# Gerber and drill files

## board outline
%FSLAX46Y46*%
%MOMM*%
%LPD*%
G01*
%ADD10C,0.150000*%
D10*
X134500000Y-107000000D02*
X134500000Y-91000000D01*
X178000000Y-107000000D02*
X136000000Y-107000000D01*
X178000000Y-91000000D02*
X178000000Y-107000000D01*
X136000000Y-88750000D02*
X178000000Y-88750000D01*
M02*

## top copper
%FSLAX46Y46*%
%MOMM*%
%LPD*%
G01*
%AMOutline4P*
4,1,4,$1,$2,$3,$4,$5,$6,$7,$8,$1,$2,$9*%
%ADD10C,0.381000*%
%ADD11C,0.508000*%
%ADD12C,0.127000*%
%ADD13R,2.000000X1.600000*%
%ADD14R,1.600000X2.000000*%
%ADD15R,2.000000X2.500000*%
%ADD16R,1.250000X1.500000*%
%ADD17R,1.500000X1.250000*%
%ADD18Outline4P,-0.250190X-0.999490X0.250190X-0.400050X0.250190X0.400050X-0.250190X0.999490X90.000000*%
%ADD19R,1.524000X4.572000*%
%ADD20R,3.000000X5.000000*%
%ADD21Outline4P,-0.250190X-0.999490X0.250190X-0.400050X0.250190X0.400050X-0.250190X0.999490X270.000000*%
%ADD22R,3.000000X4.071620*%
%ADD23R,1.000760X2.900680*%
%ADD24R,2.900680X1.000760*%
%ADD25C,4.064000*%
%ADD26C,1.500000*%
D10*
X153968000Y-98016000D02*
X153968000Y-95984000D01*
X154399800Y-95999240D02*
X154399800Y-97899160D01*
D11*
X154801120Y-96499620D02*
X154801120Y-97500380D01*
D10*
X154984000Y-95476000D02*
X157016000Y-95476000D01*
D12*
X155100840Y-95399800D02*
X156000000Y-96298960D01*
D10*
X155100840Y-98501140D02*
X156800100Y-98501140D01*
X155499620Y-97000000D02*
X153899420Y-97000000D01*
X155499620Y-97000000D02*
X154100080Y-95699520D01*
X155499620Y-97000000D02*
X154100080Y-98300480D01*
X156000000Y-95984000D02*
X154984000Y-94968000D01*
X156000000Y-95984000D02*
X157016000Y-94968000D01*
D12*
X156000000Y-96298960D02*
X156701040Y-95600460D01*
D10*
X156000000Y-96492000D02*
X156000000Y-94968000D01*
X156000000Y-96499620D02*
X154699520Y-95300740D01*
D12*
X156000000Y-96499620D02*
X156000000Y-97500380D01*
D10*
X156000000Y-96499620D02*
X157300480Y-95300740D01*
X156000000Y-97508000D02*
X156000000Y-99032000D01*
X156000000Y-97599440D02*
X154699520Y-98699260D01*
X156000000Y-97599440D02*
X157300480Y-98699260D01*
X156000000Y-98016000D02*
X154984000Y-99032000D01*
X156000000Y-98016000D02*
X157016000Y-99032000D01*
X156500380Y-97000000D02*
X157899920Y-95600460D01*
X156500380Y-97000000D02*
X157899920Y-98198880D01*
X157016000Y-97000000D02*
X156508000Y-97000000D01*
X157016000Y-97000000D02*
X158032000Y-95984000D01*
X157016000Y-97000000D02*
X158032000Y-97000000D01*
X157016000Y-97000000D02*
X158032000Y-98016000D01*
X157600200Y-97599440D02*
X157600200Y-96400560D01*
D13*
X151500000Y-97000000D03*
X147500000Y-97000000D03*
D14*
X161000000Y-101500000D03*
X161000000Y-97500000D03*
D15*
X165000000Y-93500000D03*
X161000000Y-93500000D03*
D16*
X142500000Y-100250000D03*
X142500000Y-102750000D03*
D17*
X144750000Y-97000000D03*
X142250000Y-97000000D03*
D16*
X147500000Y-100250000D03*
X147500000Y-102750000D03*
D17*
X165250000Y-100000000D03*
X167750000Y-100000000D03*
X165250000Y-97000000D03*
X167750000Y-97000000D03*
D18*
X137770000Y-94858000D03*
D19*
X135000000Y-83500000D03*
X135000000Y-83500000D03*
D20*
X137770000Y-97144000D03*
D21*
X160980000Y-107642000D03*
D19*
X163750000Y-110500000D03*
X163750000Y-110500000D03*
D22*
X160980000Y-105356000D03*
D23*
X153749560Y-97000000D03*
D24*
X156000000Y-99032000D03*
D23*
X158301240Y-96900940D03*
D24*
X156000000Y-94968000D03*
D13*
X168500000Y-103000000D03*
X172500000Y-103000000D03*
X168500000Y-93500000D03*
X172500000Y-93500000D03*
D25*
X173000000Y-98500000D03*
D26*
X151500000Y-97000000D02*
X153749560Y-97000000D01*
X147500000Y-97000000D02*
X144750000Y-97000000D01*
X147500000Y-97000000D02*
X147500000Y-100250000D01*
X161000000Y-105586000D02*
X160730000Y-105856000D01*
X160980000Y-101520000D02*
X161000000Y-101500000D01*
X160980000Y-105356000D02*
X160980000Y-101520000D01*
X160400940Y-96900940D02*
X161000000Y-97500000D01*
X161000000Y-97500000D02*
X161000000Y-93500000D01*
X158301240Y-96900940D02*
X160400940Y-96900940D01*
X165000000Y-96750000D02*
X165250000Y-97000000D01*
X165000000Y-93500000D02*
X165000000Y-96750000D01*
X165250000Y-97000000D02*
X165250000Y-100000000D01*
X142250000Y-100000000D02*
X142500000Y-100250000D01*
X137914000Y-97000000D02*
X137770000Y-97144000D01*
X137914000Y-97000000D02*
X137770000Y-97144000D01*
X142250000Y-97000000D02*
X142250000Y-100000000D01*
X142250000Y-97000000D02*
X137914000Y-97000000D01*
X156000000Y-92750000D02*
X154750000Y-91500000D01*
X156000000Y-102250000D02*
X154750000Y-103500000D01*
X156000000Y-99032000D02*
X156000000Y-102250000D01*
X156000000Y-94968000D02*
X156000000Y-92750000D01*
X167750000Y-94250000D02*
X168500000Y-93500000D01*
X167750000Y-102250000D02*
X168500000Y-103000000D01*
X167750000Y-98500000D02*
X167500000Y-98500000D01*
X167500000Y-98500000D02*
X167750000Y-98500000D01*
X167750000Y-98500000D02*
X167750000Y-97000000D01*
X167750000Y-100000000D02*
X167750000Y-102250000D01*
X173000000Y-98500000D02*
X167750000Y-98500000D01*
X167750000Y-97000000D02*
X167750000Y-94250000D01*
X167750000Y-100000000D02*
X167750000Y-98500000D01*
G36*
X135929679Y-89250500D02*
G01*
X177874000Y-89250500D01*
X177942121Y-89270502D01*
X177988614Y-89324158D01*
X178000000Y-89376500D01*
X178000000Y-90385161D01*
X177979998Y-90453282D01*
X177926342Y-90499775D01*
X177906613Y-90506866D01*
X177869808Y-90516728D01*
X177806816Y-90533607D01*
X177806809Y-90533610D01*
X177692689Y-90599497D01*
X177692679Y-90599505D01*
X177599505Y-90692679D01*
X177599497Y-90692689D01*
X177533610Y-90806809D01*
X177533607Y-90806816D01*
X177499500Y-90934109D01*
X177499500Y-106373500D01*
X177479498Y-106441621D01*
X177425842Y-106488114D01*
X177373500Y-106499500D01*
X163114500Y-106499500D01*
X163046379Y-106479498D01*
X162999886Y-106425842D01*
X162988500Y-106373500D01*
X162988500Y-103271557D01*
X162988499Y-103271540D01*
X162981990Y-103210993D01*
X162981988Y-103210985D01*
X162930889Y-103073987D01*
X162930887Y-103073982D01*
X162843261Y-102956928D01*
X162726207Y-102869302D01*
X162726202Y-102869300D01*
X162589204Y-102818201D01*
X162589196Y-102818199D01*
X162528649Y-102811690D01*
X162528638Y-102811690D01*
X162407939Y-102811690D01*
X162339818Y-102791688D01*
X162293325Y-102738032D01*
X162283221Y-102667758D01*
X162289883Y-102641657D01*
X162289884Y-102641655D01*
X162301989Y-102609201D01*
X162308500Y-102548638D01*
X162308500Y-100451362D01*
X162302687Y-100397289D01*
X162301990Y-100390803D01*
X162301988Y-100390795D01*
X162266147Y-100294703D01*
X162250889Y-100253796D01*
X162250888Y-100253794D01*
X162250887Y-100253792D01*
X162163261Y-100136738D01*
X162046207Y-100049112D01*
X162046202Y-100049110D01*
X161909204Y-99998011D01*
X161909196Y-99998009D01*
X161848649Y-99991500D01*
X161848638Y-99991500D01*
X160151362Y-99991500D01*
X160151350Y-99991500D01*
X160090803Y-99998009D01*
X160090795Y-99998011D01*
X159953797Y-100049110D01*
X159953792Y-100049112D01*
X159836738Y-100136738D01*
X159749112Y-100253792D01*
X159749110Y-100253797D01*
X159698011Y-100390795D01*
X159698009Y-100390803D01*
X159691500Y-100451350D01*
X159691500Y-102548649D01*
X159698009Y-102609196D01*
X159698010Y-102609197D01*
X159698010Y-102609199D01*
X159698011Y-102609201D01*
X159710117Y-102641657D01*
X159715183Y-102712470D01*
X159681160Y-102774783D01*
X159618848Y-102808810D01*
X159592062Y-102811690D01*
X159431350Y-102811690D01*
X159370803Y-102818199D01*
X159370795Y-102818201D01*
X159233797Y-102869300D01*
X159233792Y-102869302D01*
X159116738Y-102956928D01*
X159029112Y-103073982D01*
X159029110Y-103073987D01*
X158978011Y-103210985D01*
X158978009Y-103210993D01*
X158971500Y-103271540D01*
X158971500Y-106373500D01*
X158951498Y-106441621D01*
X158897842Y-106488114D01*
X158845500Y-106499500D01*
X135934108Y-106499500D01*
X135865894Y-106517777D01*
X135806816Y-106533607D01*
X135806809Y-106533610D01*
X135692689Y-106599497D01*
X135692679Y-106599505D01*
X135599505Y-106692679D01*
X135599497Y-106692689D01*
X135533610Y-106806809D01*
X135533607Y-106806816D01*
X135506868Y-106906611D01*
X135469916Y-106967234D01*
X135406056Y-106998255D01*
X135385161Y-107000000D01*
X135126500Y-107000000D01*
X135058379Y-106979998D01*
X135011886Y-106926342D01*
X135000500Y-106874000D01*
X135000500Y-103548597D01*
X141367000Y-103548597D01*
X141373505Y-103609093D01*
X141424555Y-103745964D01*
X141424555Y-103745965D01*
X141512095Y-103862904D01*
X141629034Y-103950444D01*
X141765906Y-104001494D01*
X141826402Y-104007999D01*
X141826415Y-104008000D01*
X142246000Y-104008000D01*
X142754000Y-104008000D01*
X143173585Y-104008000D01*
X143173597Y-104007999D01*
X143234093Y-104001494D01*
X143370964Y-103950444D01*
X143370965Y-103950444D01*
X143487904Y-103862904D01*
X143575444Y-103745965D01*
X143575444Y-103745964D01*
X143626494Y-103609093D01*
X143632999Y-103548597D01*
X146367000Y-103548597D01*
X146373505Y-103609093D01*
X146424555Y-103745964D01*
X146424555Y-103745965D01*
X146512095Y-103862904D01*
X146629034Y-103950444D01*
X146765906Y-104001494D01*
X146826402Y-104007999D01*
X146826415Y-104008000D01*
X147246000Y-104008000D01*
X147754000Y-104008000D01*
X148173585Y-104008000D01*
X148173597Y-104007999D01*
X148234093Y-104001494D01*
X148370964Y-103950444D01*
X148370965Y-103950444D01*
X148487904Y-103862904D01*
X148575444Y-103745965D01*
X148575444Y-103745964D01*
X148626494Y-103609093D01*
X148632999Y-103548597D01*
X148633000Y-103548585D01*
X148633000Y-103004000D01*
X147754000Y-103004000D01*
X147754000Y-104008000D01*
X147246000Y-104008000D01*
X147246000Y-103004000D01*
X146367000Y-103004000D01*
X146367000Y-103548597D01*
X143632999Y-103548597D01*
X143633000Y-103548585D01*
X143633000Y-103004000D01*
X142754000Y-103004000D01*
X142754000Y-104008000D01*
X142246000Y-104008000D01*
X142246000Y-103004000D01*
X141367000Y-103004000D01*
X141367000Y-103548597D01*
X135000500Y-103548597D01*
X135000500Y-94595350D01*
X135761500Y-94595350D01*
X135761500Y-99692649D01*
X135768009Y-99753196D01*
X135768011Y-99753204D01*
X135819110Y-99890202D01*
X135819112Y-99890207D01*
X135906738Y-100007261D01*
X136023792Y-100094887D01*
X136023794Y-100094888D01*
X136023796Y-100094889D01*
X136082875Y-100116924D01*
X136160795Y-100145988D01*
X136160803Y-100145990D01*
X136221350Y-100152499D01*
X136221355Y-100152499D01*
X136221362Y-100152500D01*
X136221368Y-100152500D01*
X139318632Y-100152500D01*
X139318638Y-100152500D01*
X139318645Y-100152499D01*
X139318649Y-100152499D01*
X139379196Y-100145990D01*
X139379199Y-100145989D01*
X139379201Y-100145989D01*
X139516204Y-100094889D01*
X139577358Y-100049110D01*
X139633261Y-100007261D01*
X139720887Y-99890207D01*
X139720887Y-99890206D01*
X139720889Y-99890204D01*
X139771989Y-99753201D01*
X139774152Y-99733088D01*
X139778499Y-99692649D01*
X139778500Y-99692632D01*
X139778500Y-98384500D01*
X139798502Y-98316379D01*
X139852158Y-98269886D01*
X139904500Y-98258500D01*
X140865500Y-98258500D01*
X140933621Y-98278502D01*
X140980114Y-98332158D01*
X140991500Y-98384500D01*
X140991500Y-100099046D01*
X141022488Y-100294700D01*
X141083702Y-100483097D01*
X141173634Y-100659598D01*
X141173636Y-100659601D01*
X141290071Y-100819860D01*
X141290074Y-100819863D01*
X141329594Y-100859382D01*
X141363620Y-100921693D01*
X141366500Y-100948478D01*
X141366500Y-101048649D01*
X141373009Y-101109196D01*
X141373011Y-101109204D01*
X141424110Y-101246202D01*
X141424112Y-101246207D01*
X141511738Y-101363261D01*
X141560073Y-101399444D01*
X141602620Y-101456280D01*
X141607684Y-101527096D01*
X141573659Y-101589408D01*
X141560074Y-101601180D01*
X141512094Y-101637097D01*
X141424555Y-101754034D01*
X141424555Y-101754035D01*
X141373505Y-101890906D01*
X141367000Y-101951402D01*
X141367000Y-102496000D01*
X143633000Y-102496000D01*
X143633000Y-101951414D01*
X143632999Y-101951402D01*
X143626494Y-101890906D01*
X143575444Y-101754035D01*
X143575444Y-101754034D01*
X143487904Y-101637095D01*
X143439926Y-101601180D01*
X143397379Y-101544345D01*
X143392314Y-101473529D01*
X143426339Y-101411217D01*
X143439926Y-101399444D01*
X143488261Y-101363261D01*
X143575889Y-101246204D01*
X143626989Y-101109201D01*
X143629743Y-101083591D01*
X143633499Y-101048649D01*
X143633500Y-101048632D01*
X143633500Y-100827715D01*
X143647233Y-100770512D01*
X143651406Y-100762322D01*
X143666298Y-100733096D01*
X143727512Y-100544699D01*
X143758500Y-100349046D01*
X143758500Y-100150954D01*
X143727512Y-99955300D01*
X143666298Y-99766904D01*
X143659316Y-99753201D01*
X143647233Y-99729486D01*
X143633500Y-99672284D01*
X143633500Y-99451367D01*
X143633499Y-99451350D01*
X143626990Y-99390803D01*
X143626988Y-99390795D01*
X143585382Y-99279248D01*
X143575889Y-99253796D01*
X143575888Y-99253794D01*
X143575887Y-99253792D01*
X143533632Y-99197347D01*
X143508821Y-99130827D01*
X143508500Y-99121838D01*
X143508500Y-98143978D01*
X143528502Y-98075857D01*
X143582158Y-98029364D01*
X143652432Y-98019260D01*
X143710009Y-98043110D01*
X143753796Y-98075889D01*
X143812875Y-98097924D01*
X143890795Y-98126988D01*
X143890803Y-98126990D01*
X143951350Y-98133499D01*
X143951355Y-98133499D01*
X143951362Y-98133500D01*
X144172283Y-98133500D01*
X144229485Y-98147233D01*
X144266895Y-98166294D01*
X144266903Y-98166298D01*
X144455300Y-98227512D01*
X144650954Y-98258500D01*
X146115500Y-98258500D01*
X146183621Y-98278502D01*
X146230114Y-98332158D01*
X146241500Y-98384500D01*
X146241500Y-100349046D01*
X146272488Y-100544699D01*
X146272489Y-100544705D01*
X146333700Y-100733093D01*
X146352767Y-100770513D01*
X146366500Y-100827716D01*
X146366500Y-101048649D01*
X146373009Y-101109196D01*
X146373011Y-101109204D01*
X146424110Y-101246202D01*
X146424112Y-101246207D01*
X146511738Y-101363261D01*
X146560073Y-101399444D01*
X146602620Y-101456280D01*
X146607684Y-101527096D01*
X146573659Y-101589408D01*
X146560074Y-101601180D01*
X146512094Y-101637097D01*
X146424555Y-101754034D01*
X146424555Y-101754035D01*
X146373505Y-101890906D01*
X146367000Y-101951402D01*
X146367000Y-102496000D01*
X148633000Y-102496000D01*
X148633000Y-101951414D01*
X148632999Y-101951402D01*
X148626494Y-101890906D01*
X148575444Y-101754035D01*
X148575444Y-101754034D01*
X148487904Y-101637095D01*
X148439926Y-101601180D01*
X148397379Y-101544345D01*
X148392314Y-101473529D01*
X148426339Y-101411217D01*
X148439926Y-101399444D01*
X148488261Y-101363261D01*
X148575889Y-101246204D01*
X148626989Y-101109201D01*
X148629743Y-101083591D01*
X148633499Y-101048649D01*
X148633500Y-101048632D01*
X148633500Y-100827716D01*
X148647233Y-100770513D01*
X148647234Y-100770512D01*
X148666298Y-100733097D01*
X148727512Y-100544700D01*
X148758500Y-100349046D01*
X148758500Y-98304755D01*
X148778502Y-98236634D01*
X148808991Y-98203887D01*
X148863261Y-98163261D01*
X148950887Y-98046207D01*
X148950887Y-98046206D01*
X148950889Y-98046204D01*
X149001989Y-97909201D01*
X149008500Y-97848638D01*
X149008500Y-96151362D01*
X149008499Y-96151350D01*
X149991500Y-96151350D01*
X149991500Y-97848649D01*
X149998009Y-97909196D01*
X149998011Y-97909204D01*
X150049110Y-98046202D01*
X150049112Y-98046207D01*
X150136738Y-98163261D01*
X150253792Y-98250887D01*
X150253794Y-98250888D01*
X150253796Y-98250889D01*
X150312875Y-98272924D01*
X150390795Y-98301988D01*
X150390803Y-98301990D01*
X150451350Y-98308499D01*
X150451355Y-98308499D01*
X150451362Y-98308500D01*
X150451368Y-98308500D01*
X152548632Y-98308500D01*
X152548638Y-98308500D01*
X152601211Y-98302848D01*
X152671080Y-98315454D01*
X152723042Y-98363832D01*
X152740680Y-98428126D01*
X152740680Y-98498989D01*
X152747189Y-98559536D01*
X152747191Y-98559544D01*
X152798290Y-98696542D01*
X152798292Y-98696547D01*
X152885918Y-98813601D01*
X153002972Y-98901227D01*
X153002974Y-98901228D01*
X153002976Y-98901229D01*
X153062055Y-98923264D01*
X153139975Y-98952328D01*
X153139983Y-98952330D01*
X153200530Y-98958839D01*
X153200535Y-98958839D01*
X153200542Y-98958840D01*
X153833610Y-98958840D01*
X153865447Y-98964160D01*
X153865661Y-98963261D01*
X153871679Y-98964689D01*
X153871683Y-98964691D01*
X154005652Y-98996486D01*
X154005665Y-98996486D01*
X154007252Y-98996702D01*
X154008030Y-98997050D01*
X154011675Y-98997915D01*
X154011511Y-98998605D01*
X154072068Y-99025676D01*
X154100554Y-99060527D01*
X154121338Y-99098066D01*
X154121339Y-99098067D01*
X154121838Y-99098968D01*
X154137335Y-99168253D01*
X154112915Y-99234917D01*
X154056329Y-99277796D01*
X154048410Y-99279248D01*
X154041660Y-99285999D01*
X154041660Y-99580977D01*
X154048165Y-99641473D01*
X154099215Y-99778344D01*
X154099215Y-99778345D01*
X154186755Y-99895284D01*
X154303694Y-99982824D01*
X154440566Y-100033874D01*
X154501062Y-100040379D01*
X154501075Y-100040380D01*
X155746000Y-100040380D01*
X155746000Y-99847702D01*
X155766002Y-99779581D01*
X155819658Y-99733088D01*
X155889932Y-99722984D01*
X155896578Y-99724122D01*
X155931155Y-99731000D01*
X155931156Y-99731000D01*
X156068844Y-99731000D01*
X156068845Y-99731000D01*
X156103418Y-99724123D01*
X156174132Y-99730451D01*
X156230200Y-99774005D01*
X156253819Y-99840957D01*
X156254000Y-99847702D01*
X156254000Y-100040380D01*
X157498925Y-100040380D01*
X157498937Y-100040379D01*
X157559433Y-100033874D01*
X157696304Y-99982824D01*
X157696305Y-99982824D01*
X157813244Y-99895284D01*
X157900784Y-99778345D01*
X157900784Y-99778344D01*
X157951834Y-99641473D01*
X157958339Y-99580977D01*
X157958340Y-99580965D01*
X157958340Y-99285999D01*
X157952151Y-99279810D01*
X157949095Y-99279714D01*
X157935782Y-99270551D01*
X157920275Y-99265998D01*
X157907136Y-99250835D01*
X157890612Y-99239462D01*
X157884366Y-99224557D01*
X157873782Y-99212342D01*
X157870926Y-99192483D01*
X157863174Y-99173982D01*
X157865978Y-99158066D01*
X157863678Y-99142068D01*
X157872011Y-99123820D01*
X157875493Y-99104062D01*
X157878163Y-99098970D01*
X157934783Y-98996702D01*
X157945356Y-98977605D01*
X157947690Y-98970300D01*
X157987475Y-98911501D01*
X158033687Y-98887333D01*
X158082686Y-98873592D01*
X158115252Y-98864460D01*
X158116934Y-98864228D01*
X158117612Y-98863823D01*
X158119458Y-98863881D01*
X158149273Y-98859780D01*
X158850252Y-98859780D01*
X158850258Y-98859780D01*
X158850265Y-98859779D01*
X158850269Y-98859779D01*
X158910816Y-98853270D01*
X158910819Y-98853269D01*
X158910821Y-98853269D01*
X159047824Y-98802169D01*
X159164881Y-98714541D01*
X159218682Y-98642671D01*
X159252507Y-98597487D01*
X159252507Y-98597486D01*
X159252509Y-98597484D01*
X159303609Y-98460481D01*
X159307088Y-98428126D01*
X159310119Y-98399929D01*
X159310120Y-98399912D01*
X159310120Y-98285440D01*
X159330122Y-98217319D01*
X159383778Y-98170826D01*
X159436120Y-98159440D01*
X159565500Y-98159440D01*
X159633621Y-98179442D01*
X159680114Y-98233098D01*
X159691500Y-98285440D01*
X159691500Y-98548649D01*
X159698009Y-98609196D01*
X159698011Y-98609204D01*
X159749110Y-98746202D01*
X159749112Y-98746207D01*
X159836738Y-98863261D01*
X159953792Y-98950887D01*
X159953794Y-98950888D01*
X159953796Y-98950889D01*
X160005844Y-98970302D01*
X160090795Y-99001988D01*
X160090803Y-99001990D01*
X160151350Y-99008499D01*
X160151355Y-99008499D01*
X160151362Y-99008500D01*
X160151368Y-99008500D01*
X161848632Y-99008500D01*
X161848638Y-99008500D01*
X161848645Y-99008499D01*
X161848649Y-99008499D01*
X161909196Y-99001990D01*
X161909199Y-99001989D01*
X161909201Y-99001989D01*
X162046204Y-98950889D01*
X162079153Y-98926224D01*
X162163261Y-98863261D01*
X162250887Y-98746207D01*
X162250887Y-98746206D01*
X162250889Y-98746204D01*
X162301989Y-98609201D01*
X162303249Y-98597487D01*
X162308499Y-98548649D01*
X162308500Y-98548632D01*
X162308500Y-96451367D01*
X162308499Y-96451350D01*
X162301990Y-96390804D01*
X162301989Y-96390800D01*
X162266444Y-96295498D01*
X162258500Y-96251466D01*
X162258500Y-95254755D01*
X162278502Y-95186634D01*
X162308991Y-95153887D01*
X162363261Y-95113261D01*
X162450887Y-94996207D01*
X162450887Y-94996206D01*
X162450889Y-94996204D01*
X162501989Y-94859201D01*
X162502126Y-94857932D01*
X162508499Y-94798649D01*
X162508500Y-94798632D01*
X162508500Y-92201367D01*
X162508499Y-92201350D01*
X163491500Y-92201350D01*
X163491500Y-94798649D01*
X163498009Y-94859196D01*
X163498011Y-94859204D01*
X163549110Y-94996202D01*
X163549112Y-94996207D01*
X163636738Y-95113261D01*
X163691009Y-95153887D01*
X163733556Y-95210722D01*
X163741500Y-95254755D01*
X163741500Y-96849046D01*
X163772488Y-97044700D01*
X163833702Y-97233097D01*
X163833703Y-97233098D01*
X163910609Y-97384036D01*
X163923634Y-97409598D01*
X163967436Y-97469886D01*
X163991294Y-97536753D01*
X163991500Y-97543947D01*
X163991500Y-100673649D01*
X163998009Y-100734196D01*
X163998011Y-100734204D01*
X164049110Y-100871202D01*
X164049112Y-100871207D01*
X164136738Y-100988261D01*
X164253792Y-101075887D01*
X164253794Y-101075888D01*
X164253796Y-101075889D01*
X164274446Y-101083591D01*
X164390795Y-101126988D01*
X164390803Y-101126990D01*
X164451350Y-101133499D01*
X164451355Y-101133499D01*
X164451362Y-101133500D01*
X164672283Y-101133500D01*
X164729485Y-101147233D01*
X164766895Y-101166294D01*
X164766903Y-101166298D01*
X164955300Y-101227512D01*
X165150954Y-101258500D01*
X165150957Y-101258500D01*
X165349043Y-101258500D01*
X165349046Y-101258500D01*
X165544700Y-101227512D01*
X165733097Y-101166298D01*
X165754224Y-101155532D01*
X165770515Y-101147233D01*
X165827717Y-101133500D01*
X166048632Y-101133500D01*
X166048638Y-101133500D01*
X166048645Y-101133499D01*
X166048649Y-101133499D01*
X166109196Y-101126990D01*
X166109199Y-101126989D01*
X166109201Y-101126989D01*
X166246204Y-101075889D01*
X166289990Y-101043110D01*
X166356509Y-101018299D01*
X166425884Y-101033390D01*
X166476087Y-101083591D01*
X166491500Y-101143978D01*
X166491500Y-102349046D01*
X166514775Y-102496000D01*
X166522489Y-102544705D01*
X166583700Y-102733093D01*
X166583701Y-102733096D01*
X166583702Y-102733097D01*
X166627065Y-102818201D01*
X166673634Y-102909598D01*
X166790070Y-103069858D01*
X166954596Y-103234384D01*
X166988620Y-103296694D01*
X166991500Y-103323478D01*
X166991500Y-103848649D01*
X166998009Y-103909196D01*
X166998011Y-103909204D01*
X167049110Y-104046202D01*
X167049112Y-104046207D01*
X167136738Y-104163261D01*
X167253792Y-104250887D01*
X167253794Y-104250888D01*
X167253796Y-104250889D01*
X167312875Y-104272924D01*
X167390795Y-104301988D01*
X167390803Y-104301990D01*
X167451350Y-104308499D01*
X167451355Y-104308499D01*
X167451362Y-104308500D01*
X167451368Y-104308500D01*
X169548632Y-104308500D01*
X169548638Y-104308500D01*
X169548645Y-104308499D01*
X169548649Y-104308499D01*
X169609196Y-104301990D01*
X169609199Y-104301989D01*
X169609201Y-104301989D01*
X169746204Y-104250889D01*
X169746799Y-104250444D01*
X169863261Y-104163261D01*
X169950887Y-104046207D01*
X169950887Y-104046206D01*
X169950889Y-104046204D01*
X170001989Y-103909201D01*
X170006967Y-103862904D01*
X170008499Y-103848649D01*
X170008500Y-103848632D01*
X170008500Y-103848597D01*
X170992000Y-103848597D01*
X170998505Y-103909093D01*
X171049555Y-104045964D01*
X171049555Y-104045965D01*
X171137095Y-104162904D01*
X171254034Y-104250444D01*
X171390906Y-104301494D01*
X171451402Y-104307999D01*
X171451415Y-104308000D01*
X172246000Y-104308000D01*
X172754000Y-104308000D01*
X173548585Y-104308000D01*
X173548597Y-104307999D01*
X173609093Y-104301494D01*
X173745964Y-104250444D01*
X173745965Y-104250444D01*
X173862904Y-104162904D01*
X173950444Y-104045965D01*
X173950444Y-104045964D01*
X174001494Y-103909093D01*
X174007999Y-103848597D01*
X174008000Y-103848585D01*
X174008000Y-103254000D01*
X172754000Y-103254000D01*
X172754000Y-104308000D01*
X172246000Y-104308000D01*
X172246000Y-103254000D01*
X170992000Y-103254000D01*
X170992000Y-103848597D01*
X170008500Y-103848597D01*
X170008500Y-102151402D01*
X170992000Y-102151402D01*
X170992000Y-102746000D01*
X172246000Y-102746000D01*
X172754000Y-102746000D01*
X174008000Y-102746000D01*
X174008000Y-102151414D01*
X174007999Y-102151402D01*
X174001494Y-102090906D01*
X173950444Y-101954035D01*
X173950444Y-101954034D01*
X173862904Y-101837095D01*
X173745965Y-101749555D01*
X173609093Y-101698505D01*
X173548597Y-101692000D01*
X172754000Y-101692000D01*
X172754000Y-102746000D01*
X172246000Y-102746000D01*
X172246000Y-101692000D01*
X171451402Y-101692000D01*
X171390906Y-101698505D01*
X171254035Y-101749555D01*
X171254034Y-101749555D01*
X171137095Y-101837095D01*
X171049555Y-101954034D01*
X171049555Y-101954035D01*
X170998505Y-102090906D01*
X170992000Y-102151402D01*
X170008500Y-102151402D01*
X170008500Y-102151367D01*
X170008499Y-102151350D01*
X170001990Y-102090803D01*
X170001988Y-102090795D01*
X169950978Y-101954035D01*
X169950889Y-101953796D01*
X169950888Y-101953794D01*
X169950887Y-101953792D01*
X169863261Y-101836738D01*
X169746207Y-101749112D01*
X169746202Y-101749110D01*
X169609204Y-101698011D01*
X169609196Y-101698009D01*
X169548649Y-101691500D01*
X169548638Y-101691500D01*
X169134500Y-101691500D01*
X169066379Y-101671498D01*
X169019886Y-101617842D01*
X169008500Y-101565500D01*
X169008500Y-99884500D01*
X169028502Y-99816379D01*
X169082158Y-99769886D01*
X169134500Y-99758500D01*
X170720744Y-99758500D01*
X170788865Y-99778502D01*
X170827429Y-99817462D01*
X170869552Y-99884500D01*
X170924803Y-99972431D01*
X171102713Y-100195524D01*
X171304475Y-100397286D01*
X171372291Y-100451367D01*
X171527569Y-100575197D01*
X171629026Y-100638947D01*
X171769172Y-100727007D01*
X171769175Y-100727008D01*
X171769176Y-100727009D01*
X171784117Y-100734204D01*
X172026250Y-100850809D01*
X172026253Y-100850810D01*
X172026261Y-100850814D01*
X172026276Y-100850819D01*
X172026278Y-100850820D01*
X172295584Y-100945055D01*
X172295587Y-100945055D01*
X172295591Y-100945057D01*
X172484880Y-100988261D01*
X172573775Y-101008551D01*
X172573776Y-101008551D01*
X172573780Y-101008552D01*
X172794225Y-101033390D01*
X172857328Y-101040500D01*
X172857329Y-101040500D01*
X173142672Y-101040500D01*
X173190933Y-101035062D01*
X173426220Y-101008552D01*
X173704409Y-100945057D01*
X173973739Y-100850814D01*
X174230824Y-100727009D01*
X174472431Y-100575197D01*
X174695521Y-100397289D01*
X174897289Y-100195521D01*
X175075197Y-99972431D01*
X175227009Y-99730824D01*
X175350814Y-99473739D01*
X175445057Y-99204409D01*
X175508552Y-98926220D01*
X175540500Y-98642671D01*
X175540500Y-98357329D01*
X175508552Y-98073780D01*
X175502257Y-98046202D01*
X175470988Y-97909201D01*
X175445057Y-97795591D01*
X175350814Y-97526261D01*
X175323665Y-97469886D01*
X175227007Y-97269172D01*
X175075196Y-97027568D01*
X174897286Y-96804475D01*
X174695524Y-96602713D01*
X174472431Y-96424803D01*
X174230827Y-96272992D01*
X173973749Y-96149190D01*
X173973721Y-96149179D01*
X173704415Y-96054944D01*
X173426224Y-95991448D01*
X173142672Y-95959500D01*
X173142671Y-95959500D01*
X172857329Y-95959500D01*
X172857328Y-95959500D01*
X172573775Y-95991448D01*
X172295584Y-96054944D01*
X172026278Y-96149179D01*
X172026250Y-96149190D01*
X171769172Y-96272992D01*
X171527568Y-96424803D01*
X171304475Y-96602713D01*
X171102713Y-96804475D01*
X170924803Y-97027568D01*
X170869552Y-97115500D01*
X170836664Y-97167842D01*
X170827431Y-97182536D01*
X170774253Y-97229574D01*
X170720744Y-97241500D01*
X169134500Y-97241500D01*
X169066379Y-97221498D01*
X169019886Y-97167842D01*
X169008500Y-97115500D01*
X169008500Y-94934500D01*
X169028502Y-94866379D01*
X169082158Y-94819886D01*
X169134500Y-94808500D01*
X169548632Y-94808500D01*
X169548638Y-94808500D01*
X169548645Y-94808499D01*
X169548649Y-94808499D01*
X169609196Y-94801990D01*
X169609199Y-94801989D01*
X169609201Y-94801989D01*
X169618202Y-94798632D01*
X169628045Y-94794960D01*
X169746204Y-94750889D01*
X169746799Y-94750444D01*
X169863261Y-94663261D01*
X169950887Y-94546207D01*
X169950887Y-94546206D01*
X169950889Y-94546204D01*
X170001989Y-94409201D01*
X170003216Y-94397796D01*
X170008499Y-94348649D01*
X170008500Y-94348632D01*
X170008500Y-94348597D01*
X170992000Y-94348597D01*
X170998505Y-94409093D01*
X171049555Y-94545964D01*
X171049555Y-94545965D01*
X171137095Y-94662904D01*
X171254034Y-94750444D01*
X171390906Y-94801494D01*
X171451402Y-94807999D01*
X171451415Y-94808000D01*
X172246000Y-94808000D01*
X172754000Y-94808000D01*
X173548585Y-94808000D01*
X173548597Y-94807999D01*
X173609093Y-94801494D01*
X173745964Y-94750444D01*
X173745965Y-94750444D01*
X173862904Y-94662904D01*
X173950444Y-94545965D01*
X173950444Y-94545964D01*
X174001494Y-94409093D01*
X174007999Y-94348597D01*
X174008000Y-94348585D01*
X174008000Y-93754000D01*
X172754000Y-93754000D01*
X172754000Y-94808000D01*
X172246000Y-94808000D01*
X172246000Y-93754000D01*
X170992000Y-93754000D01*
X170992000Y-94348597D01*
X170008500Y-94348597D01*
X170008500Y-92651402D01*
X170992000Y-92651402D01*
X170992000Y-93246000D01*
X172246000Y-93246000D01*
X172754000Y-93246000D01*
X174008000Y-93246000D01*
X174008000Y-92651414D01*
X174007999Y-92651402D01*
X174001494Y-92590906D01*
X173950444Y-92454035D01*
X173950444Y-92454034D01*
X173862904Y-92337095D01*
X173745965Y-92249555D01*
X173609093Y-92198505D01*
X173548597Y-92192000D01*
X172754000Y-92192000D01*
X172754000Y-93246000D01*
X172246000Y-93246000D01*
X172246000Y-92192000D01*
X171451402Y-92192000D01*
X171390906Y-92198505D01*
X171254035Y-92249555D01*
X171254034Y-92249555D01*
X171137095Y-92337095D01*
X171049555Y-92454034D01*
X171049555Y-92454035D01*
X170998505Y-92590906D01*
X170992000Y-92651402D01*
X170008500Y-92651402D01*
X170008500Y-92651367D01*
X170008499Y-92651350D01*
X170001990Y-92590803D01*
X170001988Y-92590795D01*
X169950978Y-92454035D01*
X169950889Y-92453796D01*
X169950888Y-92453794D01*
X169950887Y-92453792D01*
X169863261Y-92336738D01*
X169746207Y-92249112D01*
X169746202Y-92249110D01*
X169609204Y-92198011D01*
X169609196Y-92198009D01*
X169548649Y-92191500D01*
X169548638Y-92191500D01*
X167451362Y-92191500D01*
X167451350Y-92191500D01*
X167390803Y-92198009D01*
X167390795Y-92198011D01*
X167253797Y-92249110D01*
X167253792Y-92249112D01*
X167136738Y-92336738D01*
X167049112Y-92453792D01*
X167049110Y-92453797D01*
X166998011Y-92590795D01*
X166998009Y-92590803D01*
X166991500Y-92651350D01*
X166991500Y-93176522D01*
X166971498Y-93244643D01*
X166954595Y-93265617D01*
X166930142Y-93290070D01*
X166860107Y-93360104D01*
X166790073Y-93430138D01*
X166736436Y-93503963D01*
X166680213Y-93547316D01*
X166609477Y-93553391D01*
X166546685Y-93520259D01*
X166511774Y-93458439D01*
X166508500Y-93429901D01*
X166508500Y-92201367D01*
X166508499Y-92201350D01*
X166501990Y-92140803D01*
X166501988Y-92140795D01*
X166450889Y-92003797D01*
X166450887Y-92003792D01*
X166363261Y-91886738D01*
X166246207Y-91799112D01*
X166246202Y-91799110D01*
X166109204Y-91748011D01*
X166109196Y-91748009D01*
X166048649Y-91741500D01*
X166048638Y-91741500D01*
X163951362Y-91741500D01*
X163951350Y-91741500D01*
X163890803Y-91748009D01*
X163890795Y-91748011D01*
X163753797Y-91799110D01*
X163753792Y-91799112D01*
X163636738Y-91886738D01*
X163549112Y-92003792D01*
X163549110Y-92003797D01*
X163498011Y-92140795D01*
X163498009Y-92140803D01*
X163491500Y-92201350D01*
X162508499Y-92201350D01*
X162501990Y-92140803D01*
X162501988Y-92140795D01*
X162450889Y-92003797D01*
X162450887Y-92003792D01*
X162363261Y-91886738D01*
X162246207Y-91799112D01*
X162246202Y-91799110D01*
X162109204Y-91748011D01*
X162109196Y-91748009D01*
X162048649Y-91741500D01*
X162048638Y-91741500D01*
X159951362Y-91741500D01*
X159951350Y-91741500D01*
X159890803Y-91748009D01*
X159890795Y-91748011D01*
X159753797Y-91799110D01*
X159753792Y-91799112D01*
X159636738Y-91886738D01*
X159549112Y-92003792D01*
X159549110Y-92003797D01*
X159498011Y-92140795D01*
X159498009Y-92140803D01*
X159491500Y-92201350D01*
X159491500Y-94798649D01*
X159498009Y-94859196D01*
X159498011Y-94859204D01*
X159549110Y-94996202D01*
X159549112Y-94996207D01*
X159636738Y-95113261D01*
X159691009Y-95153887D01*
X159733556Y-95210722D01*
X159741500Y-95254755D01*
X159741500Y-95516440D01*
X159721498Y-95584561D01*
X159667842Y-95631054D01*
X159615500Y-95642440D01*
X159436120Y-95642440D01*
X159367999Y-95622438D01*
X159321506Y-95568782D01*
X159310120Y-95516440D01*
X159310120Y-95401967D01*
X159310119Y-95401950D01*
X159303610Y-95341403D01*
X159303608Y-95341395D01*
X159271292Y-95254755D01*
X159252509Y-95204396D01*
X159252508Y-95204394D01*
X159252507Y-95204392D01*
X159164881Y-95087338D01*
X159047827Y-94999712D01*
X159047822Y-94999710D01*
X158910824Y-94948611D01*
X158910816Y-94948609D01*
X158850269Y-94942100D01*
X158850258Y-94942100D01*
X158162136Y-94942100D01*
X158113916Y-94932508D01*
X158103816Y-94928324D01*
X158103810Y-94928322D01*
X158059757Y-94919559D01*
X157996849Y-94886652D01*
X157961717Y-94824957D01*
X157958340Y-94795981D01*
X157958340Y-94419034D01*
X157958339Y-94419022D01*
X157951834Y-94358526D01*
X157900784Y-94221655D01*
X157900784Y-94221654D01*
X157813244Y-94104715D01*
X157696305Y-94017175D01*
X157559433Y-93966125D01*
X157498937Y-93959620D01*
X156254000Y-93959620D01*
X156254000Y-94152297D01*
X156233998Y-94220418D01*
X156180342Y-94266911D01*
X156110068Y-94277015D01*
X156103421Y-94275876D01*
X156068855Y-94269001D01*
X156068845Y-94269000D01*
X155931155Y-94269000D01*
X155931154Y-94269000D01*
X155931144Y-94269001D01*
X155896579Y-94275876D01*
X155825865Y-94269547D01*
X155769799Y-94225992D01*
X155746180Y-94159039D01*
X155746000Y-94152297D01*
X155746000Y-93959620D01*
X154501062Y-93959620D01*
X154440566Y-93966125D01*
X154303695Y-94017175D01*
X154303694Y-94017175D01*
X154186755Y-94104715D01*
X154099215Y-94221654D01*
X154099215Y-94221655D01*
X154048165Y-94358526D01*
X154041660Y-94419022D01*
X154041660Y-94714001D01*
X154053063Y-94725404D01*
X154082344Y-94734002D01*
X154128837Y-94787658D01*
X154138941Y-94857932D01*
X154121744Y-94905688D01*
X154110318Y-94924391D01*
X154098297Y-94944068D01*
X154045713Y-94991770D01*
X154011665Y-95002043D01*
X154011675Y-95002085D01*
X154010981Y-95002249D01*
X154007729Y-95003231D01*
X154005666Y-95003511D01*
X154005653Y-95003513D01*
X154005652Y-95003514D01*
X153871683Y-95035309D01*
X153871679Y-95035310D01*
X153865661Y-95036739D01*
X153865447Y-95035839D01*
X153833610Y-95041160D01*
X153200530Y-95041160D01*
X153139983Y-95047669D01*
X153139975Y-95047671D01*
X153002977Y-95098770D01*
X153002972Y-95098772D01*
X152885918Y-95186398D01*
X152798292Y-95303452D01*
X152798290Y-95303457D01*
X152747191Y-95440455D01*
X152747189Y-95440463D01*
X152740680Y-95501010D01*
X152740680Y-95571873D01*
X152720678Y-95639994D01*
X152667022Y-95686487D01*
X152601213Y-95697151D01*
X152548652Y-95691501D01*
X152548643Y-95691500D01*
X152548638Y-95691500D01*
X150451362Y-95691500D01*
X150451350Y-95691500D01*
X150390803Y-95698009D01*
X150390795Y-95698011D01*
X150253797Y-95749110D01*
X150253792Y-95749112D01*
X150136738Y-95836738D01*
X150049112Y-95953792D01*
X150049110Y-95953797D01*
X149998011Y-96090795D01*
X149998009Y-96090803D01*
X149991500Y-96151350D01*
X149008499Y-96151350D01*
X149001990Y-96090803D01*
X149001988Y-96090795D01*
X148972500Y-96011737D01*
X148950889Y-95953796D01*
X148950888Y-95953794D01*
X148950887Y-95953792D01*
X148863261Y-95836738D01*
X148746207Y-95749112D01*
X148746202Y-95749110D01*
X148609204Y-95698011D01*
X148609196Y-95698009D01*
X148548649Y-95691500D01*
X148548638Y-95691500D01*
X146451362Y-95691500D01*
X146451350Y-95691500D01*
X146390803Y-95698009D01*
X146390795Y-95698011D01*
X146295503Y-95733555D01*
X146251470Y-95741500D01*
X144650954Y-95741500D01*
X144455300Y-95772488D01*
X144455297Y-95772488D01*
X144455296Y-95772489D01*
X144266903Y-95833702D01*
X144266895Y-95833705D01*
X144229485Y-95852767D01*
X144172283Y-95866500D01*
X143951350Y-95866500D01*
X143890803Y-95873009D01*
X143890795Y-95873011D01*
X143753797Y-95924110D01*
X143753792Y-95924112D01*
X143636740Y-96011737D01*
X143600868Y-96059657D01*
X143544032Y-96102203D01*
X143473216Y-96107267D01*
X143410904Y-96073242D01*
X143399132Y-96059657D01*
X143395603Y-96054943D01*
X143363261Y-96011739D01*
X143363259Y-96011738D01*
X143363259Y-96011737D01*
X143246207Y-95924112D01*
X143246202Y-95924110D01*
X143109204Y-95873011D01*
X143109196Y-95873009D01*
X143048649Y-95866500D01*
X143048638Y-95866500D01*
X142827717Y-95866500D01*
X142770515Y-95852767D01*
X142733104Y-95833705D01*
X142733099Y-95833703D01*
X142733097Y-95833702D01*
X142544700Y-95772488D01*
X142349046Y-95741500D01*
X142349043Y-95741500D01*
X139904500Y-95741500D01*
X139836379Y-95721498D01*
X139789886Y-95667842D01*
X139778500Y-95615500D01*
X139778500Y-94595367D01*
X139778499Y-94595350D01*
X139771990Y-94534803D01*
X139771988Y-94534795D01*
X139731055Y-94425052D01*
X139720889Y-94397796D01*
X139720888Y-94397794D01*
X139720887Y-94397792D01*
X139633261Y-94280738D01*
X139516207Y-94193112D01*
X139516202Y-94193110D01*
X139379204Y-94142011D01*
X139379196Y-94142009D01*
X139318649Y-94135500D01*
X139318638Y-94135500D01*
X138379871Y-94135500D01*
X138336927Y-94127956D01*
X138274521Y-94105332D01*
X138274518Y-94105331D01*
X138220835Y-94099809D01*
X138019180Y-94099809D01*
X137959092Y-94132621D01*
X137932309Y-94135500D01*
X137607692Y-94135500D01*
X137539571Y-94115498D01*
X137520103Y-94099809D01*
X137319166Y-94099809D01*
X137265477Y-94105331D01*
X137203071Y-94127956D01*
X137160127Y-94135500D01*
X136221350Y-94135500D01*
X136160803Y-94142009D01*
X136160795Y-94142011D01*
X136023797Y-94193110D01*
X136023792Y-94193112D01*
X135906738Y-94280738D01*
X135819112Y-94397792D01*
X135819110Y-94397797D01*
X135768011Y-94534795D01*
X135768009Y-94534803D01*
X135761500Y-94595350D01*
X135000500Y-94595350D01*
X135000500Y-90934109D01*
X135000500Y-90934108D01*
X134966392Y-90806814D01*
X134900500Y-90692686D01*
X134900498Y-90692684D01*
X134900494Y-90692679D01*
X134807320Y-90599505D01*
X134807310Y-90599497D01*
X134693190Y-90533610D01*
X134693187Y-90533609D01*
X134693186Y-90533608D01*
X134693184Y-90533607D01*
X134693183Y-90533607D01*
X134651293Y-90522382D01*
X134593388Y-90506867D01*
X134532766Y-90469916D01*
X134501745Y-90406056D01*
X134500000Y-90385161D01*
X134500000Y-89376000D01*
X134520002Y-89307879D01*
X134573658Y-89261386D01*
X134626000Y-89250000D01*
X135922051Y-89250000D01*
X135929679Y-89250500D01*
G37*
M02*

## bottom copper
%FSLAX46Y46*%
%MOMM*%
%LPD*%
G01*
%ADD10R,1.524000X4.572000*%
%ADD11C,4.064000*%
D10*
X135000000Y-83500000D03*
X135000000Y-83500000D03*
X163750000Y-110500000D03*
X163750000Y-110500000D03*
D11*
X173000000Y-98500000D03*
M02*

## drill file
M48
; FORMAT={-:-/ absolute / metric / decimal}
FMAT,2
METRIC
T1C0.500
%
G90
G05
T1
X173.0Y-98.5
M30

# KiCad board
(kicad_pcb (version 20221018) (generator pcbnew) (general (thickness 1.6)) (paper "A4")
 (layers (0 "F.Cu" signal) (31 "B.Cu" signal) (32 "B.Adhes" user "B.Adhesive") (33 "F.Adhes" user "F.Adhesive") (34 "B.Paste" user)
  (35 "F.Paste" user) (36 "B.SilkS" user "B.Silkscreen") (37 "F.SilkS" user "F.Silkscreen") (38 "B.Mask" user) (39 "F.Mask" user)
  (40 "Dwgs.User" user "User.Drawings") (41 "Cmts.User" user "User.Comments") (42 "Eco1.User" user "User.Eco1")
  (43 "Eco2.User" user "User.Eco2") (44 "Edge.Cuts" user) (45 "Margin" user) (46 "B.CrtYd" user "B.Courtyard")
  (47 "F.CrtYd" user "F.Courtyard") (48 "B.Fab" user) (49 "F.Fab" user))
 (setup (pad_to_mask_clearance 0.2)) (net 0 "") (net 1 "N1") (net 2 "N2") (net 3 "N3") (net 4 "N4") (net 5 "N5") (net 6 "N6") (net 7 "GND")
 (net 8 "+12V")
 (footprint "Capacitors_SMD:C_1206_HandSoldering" (layer "F.Cu") (at 149.5 97 180)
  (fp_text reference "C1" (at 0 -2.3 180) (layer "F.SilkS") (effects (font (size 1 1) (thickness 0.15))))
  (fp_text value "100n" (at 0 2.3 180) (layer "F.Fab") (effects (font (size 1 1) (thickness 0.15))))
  (pad "1" smd rect (at -2 0 180) (size 2 1.6) (layers "F.Cu" "F.Paste" "F.Mask") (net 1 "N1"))
  (pad "2" smd rect (at 2 0 180) (size 2 1.6) (layers "F.Cu" "F.Paste" "F.Mask") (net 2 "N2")))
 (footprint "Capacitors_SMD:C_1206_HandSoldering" (layer "F.Cu") (at 161 99.5 90)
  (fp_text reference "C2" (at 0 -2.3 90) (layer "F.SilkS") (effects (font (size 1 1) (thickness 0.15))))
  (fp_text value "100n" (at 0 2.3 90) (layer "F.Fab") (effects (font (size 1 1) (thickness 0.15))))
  (pad "1" smd rect (at -2 0 90) (size 2 1.6) (layers "F.Cu" "F.Paste" "F.Mask") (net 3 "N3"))
  (pad "2" smd rect (at 2 0 90) (size 2 1.6) (layers "F.Cu" "F.Paste" "F.Mask") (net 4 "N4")))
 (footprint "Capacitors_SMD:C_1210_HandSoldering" (layer "F.Cu") (at 163 93.5 180)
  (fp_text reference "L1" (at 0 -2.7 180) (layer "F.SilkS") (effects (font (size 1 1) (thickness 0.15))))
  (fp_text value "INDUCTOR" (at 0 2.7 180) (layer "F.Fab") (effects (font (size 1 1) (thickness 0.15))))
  (pad "1" smd rect (at -2 0 180) (size 2 2.5) (layers "F.Cu" "F.Paste" "F.Mask") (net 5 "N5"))
  (pad "2" smd rect (at 2 0 180) (size 2 2.5) (layers "F.Cu" "F.Paste" "F.Mask") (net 4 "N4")))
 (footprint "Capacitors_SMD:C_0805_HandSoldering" (layer "F.Cu") (at 142.5 101.5 -90)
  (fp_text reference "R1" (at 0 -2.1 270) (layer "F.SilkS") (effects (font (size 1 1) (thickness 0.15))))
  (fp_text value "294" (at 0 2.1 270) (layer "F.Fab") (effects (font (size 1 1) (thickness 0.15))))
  (pad "1" smd rect (at -1.25 0 270) (size 1.5 1.25) (layers "F.Cu" "F.Paste" "F.Mask") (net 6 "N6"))
  (pad "2" smd rect (at 1.25 0 270) (size 1.5 1.25) (layers "F.Cu" "F.Paste" "F.Mask") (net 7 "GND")))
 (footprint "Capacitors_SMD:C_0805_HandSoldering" (layer "F.Cu") (at 143.5 97 180)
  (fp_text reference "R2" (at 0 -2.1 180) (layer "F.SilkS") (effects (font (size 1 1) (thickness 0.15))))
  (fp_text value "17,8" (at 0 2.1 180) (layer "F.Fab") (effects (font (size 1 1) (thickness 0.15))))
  (pad "1" smd rect (at -1.25 0 180) (size 1.5 1.25) (layers "F.Cu" "F.Paste" "F.Mask") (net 2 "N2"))
  (pad "2" smd rect (at 1.25 0 180) (size 1.5 1.25) (layers "F.Cu" "F.Paste" "F.Mask") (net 6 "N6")))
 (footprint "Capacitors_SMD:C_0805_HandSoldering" (layer "F.Cu") (at 147.5 101.5 -90)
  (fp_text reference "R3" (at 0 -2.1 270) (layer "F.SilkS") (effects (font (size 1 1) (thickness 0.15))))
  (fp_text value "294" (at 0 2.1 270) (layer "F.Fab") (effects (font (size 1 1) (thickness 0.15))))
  (pad "1" smd rect (at -1.25 0 270) (size 1.5 1.25) (layers "F.Cu" "F.Paste" "F.Mask") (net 2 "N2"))
  (pad "2" smd rect (at 1.25 0 270) (size 1.5 1.25) (layers "F.Cu" "F.Paste" "F.Mask") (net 7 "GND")))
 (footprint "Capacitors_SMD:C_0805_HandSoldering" (layer "F.Cu") (at 166.5 100)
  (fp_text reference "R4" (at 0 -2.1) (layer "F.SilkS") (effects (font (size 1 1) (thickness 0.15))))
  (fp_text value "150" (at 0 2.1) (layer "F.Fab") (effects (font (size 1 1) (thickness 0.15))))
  (pad "1" smd rect (at -1.25 0) (size 1.5 1.25) (layers "F.Cu" "F.Paste" "F.Mask") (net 5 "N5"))
  (pad "2" smd rect (at 1.25 0) (size 1.5 1.25) (layers "F.Cu" "F.Paste" "F.Mask") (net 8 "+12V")))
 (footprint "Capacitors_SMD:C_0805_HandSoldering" (layer "F.Cu") (at 166.5 97)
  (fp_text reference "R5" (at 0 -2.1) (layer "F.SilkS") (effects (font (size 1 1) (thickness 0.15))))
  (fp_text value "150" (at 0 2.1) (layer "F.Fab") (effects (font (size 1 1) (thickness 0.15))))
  (pad "1" smd rect (at -1.25 0) (size 1.5 1.25) (layers "F.Cu" "F.Paste" "F.Mask") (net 5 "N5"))
  (pad "2" smd rect (at 1.25 0) (size 1.5 1.25) (layers "F.Cu" "F.Paste" "F.Mask") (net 8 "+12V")))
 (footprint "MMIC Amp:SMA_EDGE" (layer "F.Cu") (at 136.5 88 90)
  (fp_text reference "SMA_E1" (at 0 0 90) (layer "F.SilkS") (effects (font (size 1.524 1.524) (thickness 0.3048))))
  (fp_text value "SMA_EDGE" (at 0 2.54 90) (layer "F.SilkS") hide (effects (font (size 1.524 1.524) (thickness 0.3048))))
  (pad "1" connect trapezoid (at -6.858 1.27 90) (size 0.50038 1.39954) (rect_delta 0.59944 0) (layers "F.Cu" "F.Mask") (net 7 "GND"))
  (pad "1" connect rect (at 4.5 -1.5 90) (size 4.572 1.524) (layers "*.Cu" "F.Mask") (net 7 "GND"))
  (pad "2" connect rect (at 4.5 -1.5 90) (size 4.572 1.524) (layers "*.Cu" "F.Mask") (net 7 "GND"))
  (pad "3" connect rect (at -9.144 1.27 90) (size 5 3) (layers "F.Cu" "F.Mask") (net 6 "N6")))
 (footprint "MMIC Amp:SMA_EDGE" (layer "F.Cu") (at 162.25 114.5 -90)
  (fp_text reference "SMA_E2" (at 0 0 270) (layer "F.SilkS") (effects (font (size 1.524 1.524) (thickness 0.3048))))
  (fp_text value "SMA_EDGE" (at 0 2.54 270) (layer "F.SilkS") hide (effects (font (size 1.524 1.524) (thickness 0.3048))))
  (pad "1" connect trapezoid (at -6.858 1.27 270) (size 0.50038 1.39954) (rect_delta 0.59944 0) (layers "F.Cu" "F.Mask") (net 7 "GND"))
  (pad "1" connect rect (at -4 -1.5 270) (size 4.572 1.524) (layers "*.Cu" "F.Mask") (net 7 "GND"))
  (pad "2" connect rect (at -4 -1.5 270) (size 4.572 1.524) (layers "*.Cu" "F.Mask") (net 7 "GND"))
  (pad "3" connect rect (at -9.144 1.27 270) (size 4.07162 3) (layers "F.Cu" "F.Mask") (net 3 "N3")))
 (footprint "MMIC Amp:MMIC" (layer "F.Cu") (at 156 97)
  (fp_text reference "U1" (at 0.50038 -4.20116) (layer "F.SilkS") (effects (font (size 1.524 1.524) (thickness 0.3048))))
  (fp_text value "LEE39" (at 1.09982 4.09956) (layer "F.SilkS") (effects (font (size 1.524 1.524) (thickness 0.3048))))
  (fp_line (start -2.032 1.016) (end -2.032 -1.016) (stroke (width 0.381) (type solid)) (layer "F.Cu"))
  (fp_line (start -1.6002 -1.00076) (end -1.6002 0.89916) (stroke (width 0.381) (type solid)) (layer "F.Cu"))
  (fp_line (start -1.19888 -0.50038) (end -1.19888 0.50038) (stroke (width 0.508) (type solid)) (layer "F.Cu"))
  (fp_line (start -1.016 -1.524) (end 1.016 -1.524) (stroke (width 0.381) (type solid)) (layer "F.Cu"))
  (fp_line (start -0.89916 -1.6002) (end 0 -0.70104) (stroke (width 0.127) (type solid)) (layer "F.Cu"))
  (fp_line (start -0.89916 1.50114) (end 0.8001 1.50114) (stroke (width 0.381) (type solid)) (layer "F.Cu"))
  (fp_line (start -0.50038 0) (end -2.10058 0) (stroke (width 0.381) (type solid)) (layer "F.Cu"))
  (fp_line (start -0.50038 0) (end -1.89992 -1.30048) (stroke (width 0.381) (type solid)) (layer "F.Cu"))
  (fp_line (start -0.50038 0) (end -1.89992 1.30048) (stroke (width 0.381) (type solid)) (layer "F.Cu"))
  (fp_line (start 0 -1.016) (end -1.016 -2.032) (stroke (width 0.381) (type solid)) (layer "F.Cu"))
  (fp_line (start 0 -1.016) (end 1.016 -2.032) (stroke (width 0.381) (type solid)) (layer "F.Cu"))
  (fp_line (start 0 -0.70104) (end 0.70104 -1.39954) (stroke (width 0.127) (type solid)) (layer "F.Cu"))
  (fp_line (start 0 -0.508) (end 0 -2.032) (stroke (width 0.381) (type solid)) (layer "F.Cu"))
  (fp_line (start 0 -0.50038) (end -1.30048 -1.69926) (stroke (width 0.381) (type solid)) (layer "F.Cu"))
  (fp_line (start 0 -0.50038) (end 0 0.50038) (stroke (width 0.127) (type solid)) (layer "F.Cu"))
  (fp_line (start 0 -0.50038) (end 1.30048 -1.69926) (stroke (width 0.381) (type solid)) (layer "F.Cu"))
  (fp_line (start 0 0.508) (end 0 2.032) (stroke (width 0.381) (type solid)) (layer "F.Cu"))
  (fp_line (start 0 0.59944) (end -1.30048 1.69926) (stroke (width 0.381) (type solid)) (layer "F.Cu"))
  (fp_line (start 0 0.59944) (end 1.30048 1.69926) (stroke (width 0.381) (type solid)) (layer "F.Cu"))
  (fp_line (start 0 1.016) (end -1.016 2.032) (stroke (width 0.381) (type solid)) (layer "F.Cu"))
  (fp_line (start 0 1.016) (end 1.016 2.032) (stroke (width 0.381) (type solid)) (layer "F.Cu"))
  (fp_line (start 0.50038 0) (end 1.89992 -1.39954) (stroke (width 0.381) (type solid)) (layer "F.Cu"))
  (fp_line (start 0.50038 0) (end 1.89992 1.19888) (stroke (width 0.381) (type solid)) (layer "F.Cu"))
  (fp_line (start 1.016 0) (end 0.508 0) (stroke (width 0.381) (type solid)) (layer "F.Cu"))
  (fp_line (start 1.016 0) (end 2.032 -1.016) (stroke (width 0.381) (type solid)) (layer "F.Cu"))
  (fp_line (start 1.016 0) (end 2.032 0) (stroke (width 0.381) (type solid)) (layer "F.Cu"))
  (fp_line (start 1.016 0) (end 2.032 1.016) (stroke (width 0.381) (type solid)) (layer "F.Cu"))
  (fp_line (start 1.6002 0.59944) (end 1.6002 -0.59944) (stroke (width 0.381) (type solid)) (layer "F.Cu"))
  (pad "1" smd rect (at -2.25044 0) (size 1.00076 2.90068) (layers "F.Cu" "F.Paste" "F.Mask") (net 1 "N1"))
  (pad "2" smd rect (at 0 2.032) (size 2.90068 1.00076) (layers "F.Cu" "F.Paste" "F.Mask") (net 7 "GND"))
  (pad "3" smd rect (at 2.30124 -0.09906) (size 1.00076 2.90068) (layers "F.Cu" "F.Paste" "F.Mask") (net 4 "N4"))
  (pad "4" smd rect (at 0 -2.032) (size 2.90068 1.00076) (layers "F.Cu" "F.Paste" "F.Mask") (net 7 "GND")))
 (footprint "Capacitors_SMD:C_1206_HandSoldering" (layer "F.Cu") (at 170.5 103)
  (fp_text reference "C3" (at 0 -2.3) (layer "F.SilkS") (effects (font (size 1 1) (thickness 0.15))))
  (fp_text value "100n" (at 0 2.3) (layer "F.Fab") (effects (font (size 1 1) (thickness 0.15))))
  (pad "1" smd rect (at -2 0) (size 2 1.6) (layers "F.Cu" "F.Paste" "F.Mask") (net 8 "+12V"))
  (pad "2" smd rect (at 2 0) (size 2 1.6) (layers "F.Cu" "F.Paste" "F.Mask") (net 7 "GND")))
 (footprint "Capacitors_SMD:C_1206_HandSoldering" (layer "F.Cu") (at 170.5 93.5)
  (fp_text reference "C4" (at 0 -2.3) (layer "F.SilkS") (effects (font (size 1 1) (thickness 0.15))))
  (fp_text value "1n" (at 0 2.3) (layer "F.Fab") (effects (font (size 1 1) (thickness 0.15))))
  (pad "1" smd rect (at -2 0) (size 2 1.6) (layers "F.Cu" "F.Paste" "F.Mask") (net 8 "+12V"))
  (pad "2" smd rect (at 2 0) (size 2 1.6) (layers "F.Cu" "F.Paste" "F.Mask") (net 7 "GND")))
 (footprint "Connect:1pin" (layer "F.Cu") (at 173 98.5)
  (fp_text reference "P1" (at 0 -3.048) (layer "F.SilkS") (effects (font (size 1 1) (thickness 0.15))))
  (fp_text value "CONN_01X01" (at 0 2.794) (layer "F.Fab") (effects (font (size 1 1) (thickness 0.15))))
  (pad "1" thru_hole circle (at 0 0) (size 4.064 4.064) (drill 0.5) (layers "*.Cu" "*.Mask" "F.SilkS") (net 8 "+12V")))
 (gr_line (start 134.5 107) (end 134.5 91) (stroke (width 0.15) (type solid)) (layer "Edge.Cuts"))
 (gr_line (start 178 107) (end 136 107) (stroke (width 0.15) (type solid)) (layer "Edge.Cuts"))
 (gr_line (start 178 91) (end 178 107) (stroke (width 0.15) (type solid)) (layer "Edge.Cuts"))
 (gr_line (start 136 88.75) (end 178 88.75) (stroke (width 0.15) (type solid)) (layer "Edge.Cuts"))
 (segment (start 151.5 97) (end 153.74956 97) (width 1.5) (layer "F.Cu") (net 1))
 (segment (start 147.5 97) (end 144.75 97) (width 1.5) (layer "F.Cu") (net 2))
 (segment (start 147.5 97) (end 147.5 100.25) (width 1.5) (layer "F.Cu") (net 2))
 (segment (start 161 105.586) (end 160.73 105.856) (width 1.5) (layer "F.Cu") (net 3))
 (segment (start 160.98 101.52) (end 161 101.5) (width 1.5) (layer "F.Cu") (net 3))
 (segment (start 160.98 105.356) (end 160.98 101.52) (width 1.5) (layer "F.Cu") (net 3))
 (segment (start 160.40094 96.90094) (end 161 97.5) (width 1.5) (layer "F.Cu") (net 4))
 (segment (start 161 97.5) (end 161 93.5) (width 1.5) (layer "F.Cu") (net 4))
 (segment (start 158.30124 96.90094) (end 160.40094 96.90094) (width 1.5) (layer "F.Cu") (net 4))
 (segment (start 165 96.75) (end 165.25 97) (width 1.5) (layer "F.Cu") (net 5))
 (segment (start 165 93.5) (end 165 96.75) (width 1.5) (layer "F.Cu") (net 5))
 (segment (start 165.25 97) (end 165.25 100) (width 1.5) (layer "F.Cu") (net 5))
 (segment (start 142.25 100) (end 142.5 100.25) (width 1.5) (layer "F.Cu") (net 6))
 (segment (start 137.914 97) (end 137.77 97.144) (width 1.5) (layer "F.Cu") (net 6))
 (segment (start 137.914 97) (end 137.77 97.144) (width 1.5) (layer "F.Cu") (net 6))
 (segment (start 142.25 97) (end 142.25 100) (width 1.5) (layer "F.Cu") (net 6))
 (segment (start 142.25 97) (end 137.914 97) (width 1.5) (layer "F.Cu") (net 6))
 (segment (start 156 92.75) (end 154.75 91.5) (width 1.5) (layer "F.Cu") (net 7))
 (segment (start 156 102.25) (end 154.75 103.5) (width 1.5) (layer "F.Cu") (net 7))
 (segment (start 156 99.032) (end 156 102.25) (width 1.5) (layer "F.Cu") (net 7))
 (segment (start 156 94.968) (end 156 92.75) (width 1.5) (layer "F.Cu") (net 7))
 (segment (start 167.75 94.25) (end 168.5 93.5) (width 1.5) (layer "F.Cu") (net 8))
 (segment (start 167.75 102.25) (end 168.5 103) (width 1.5) (layer "F.Cu") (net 8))
 (segment (start 167.75 98.5) (end 167.5 98.5) (width 1.5) (layer "F.Cu") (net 8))
 (segment (start 167.5 98.5) (end 167.75 98.5) (width 1.5) (layer "F.Cu") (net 8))
 (segment (start 167.75 98.5) (end 167.75 97) (width 1.5) (layer "F.Cu") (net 8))
 (segment (start 167.75 100) (end 167.75 102.25) (width 1.5) (layer "F.Cu") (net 8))
 (segment (start 173 98.5) (end 167.75 98.5) (width 1.5) (layer "F.Cu") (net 8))
 (segment (start 167.75 97) (end 167.75 94.25) (width 1.5) (layer "F.Cu") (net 8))
 (segment (start 167.75 100) (end 167.75 98.5) (width 1.5) (layer "F.Cu") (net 8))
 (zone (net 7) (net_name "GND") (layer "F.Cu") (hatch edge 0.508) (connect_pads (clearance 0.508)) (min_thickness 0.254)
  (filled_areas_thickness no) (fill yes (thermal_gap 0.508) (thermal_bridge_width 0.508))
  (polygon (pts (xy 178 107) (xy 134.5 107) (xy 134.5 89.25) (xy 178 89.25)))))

